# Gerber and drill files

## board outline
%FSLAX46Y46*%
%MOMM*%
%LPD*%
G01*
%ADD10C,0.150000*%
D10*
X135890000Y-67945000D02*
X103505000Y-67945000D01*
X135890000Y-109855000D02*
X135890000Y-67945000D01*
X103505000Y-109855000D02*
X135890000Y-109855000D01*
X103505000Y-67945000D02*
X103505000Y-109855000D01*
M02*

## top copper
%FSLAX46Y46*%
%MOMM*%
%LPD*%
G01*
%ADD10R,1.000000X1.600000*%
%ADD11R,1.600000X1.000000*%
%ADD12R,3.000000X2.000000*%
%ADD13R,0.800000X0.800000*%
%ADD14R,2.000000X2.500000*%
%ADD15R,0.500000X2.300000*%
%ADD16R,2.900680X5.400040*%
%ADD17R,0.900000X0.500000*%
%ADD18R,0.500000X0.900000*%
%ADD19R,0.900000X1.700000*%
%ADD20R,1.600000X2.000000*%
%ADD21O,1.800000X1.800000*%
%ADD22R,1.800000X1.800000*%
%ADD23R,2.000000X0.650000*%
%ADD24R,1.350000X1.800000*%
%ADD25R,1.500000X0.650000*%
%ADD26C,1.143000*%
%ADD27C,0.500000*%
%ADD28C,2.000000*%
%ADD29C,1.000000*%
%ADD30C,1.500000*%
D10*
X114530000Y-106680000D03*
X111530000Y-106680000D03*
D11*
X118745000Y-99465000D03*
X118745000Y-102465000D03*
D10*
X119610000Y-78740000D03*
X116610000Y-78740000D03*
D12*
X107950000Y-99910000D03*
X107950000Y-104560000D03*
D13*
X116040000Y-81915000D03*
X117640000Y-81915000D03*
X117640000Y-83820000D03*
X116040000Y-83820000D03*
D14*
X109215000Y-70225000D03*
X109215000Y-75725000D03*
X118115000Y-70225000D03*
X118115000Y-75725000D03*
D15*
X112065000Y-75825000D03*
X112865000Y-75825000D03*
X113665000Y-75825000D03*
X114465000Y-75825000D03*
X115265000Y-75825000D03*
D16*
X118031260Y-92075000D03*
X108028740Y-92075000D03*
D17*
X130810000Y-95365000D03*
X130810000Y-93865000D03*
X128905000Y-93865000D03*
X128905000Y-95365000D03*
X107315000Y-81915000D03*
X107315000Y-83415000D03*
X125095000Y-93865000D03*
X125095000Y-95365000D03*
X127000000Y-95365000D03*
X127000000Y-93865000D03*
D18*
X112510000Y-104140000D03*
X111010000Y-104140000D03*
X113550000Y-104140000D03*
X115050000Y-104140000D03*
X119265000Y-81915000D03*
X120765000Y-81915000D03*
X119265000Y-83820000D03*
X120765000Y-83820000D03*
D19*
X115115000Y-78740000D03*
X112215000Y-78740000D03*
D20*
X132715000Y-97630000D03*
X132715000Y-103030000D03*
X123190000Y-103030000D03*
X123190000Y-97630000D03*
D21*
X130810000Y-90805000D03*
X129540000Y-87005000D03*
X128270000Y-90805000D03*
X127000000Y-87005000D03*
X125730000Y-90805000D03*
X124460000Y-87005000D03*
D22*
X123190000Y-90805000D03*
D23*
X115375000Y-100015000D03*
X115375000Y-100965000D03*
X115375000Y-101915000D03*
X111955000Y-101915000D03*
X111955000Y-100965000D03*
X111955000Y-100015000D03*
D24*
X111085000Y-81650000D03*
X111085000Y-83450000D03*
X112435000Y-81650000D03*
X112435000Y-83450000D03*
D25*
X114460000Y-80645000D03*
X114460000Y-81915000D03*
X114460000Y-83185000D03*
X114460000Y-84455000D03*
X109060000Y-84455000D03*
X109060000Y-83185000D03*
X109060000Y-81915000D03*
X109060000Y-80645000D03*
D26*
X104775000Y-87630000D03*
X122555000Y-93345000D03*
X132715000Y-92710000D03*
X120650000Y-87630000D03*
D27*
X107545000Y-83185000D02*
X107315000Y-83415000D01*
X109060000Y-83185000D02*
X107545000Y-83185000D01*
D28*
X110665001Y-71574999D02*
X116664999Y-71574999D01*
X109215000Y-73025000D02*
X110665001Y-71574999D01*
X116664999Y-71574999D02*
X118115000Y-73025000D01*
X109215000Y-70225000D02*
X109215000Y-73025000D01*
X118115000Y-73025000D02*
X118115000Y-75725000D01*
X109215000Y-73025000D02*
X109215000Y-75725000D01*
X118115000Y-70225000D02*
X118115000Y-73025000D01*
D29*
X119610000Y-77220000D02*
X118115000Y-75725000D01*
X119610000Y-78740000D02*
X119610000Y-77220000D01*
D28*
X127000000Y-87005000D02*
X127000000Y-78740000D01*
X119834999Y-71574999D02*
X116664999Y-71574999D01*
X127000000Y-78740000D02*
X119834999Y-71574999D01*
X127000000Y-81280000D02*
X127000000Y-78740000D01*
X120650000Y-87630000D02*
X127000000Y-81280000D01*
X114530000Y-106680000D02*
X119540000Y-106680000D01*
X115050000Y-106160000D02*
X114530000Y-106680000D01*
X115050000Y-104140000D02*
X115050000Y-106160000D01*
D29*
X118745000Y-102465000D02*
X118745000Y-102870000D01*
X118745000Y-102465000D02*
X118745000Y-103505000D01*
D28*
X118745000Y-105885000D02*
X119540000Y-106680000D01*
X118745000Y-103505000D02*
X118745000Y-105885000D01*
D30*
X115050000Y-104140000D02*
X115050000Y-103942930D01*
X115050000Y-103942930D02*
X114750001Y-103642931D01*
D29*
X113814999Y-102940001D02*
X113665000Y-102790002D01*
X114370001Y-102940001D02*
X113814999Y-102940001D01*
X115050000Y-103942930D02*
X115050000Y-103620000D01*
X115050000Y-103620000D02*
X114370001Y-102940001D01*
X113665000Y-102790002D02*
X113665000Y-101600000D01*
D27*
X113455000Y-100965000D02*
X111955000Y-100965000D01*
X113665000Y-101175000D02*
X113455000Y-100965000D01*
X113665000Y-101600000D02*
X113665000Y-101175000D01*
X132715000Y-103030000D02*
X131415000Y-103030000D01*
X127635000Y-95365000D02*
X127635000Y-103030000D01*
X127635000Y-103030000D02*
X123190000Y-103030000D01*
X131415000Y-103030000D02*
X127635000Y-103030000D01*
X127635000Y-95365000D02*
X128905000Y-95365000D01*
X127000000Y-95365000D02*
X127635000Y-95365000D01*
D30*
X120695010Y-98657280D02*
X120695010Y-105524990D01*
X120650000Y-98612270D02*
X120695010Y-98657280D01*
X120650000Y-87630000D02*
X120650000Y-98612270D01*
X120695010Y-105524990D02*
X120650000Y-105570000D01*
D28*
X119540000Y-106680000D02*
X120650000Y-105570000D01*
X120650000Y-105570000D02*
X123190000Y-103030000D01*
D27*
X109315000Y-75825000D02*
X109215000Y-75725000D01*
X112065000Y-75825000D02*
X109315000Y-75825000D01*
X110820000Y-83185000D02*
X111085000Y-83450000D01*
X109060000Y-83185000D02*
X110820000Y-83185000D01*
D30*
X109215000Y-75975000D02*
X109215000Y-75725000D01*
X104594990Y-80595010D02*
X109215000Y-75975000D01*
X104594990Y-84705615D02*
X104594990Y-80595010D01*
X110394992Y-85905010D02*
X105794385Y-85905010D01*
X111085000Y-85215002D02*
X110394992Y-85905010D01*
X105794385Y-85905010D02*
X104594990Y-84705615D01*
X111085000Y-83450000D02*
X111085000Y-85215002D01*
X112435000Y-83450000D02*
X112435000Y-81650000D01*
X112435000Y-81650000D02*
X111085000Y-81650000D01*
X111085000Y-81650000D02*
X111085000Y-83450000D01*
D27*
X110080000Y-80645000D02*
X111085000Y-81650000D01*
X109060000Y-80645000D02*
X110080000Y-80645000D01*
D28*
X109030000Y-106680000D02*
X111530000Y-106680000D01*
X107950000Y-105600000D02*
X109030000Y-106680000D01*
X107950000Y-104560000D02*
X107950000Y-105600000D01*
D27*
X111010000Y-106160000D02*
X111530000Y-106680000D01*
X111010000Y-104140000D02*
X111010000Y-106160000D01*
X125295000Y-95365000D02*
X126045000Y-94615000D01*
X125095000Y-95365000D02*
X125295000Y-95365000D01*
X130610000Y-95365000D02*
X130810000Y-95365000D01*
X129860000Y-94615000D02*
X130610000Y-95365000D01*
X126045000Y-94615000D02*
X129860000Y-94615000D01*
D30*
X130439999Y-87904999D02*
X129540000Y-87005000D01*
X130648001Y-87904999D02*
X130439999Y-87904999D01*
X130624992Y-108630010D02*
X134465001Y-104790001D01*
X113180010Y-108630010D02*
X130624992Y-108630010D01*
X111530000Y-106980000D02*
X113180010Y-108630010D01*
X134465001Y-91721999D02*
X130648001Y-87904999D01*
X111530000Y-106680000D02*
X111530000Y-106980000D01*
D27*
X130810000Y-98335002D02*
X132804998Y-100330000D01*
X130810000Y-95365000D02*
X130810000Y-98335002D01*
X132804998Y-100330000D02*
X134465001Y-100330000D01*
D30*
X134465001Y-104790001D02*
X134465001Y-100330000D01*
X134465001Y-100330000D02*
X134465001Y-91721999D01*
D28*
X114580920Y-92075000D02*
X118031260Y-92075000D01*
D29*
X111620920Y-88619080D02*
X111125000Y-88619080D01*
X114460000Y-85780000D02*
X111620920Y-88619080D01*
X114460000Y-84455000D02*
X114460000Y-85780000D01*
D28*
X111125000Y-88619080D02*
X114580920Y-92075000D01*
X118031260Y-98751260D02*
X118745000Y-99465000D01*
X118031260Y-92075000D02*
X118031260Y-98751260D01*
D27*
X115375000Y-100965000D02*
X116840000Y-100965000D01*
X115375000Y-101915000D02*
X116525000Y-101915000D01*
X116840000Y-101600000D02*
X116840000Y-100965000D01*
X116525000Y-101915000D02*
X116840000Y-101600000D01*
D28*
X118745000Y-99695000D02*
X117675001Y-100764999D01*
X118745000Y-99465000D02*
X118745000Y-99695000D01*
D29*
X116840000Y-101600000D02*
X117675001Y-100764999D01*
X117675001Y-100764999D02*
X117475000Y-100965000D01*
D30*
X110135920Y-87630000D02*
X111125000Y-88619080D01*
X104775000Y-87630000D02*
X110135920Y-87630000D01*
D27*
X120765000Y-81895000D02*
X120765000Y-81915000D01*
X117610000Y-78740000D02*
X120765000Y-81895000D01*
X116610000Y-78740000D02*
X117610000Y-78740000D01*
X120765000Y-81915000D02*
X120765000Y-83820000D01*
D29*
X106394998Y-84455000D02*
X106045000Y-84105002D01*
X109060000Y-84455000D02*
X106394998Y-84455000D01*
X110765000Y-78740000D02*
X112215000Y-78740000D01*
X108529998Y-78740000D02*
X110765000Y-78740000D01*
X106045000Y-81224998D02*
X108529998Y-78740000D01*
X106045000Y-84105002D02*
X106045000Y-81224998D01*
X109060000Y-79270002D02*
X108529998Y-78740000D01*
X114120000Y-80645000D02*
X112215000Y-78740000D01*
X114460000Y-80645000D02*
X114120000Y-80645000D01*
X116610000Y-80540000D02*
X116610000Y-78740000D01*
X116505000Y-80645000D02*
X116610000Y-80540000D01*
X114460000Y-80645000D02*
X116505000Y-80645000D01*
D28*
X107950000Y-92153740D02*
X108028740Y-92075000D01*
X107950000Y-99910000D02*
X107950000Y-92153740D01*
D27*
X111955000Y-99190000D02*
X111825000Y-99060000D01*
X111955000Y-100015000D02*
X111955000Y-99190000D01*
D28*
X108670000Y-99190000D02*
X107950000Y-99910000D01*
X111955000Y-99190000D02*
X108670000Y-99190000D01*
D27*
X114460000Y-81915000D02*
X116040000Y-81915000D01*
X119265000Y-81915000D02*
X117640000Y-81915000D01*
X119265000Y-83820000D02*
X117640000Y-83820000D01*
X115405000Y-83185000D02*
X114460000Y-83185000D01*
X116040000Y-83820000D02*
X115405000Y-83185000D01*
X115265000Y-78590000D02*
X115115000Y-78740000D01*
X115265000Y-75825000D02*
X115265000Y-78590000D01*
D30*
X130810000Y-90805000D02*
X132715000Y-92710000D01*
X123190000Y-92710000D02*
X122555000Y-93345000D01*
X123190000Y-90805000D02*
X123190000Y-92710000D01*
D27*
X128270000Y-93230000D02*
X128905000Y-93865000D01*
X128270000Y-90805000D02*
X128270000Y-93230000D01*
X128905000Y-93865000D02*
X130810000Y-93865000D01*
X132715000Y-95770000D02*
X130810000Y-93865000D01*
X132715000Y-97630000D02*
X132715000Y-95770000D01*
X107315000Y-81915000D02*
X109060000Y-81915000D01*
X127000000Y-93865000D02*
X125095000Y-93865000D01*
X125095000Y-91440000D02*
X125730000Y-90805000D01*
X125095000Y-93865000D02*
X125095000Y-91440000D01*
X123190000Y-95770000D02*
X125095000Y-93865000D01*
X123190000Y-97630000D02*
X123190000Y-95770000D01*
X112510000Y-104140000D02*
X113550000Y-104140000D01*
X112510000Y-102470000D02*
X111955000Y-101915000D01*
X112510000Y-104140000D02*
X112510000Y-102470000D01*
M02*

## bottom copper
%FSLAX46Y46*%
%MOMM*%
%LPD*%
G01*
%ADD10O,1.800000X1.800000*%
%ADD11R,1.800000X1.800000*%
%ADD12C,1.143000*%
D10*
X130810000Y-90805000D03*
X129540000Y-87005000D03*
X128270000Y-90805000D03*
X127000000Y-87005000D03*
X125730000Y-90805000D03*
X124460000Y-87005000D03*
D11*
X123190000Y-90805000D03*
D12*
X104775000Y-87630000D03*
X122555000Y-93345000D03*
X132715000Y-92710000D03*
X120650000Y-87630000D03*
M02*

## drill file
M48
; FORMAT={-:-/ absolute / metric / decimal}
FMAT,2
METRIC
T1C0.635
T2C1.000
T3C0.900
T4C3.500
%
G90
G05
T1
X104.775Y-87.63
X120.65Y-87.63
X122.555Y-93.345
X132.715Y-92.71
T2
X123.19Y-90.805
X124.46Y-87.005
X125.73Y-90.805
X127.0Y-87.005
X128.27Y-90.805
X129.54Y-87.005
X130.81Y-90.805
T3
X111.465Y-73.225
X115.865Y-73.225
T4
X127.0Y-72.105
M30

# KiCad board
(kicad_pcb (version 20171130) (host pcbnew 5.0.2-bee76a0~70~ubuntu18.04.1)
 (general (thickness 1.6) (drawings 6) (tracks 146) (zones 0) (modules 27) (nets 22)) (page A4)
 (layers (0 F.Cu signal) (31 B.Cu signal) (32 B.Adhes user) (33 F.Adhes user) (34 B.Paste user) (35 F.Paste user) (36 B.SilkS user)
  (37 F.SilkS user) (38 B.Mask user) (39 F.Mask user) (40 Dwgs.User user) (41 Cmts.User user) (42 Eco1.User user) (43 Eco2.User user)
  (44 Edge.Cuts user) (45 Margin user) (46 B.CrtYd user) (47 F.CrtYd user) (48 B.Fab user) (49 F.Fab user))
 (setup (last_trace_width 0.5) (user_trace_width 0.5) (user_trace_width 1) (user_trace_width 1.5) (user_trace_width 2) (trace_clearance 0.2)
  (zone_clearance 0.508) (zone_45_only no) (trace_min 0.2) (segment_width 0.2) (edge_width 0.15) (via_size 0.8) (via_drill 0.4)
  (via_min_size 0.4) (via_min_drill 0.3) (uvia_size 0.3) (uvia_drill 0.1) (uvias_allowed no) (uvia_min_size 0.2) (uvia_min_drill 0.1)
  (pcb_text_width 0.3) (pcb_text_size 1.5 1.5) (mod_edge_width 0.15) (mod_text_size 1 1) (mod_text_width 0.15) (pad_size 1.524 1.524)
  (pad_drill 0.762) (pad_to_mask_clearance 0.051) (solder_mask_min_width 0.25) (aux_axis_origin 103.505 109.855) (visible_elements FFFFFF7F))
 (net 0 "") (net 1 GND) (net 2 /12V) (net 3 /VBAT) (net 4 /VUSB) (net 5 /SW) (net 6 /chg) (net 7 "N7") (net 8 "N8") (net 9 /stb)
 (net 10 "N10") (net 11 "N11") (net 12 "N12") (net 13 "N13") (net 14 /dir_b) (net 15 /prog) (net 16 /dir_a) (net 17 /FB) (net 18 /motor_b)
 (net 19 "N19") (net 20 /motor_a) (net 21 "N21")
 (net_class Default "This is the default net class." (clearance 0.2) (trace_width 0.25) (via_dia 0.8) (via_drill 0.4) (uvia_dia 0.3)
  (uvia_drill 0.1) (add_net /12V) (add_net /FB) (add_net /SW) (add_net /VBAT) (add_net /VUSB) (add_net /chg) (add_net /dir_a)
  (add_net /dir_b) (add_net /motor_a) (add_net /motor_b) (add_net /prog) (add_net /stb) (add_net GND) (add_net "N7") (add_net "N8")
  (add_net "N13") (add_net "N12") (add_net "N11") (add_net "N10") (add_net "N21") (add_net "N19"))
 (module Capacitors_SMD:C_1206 (layer F.Cu) (at 113.03 106.68)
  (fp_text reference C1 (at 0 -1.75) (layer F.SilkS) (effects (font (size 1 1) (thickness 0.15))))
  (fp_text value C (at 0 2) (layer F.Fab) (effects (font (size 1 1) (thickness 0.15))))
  (pad 2 smd rect (at 1.5 0) (size 1 1.6) (layers F.Cu F.Paste F.Mask) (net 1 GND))
  (pad 1 smd rect (at -1.5 0) (size 1 1.6) (layers F.Cu F.Paste F.Mask) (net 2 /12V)))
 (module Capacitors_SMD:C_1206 (layer F.Cu) (at 118.745 100.965 270)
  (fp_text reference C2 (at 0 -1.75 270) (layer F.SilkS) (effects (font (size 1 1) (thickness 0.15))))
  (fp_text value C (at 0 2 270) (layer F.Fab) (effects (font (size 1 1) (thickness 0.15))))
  (pad 1 smd rect (at -1.5 0 270) (size 1 1.6) (layers F.Cu F.Paste F.Mask) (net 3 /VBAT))
  (pad 2 smd rect (at 1.5 0 270) (size 1 1.6) (layers F.Cu F.Paste F.Mask) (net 1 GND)))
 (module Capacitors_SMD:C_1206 (layer F.Cu) (at 118.11 78.74)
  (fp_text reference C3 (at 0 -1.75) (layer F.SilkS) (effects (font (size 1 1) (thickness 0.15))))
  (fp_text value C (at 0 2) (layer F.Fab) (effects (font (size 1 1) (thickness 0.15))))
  (pad 2 smd rect (at 1.5 0) (size 1 1.6) (layers F.Cu F.Paste F.Mask) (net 1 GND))
  (pad 1 smd rect (at -1.5 0) (size 1 1.6) (layers F.Cu F.Paste F.Mask) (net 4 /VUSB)))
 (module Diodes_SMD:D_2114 (layer F.Cu) (at 107.95 102.235 90)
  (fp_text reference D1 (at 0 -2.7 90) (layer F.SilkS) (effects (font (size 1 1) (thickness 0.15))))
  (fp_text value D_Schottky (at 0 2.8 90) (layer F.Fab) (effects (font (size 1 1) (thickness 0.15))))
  (pad 2 smd rect (at 2.325 0 90) (size 2 3) (layers F.Cu F.Paste F.Mask) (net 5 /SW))
  (pad 1 smd rect (at -2.325 0 90) (size 2 3) (layers F.Cu F.Paste F.Mask) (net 2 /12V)))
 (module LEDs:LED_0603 (layer F.Cu) (at 116.84 81.915)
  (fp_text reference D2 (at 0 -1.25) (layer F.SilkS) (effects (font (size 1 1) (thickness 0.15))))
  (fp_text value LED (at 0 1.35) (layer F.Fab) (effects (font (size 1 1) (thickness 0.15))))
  (pad 1 smd rect (at -0.8 0 180) (size 0.8 0.8) (layers F.Cu F.Paste F.Mask) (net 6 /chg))
  (pad 2 smd rect (at 0.8 0 180) (size 0.8 0.8) (layers F.Cu F.Paste F.Mask) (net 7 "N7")))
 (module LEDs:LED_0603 (layer F.Cu) (at 116.84 83.82)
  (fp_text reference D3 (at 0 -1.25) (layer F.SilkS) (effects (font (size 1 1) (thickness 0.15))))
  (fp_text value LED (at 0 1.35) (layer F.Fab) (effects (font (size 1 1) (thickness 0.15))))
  (pad 2 smd rect (at 0.8 0 180) (size 0.8 0.8) (layers F.Cu F.Paste F.Mask) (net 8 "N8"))
  (pad 1 smd rect (at -0.8 0 180) (size 0.8 0.8) (layers F.Cu F.Paste F.Mask) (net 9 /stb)))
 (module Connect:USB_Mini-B (layer F.Cu) (at 113.665 73.025 270)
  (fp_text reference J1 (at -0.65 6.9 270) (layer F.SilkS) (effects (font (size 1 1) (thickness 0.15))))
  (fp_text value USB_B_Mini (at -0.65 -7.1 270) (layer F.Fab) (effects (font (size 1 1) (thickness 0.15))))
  (pad "" np_thru_hole circle (at 0.2 2.2 270) (size 0.9 0.9) (drill 0.9) (layers *.Cu *.Mask))
  (pad "" np_thru_hole circle (at 0.2 -2.2 270) (size 0.9 0.9) (drill 0.9) (layers *.Cu *.Mask))
  (pad 6 smd rect (at -2.8 4.45 270) (size 2.5 2) (layers F.Cu F.Paste F.Mask) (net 1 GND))
  (pad 6 smd rect (at 2.7 4.45 270) (size 2.5 2) (layers F.Cu F.Paste F.Mask) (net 1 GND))
  (pad 6 smd rect (at -2.8 -4.45 270) (size 2.5 2) (layers F.Cu F.Paste F.Mask) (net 1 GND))
  (pad 6 smd rect (at 2.7 -4.45 270) (size 2.5 2) (layers F.Cu F.Paste F.Mask) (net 1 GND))
  (pad 5 smd rect (at 2.8 1.6 270) (size 2.3 0.5) (layers F.Cu F.Paste F.Mask) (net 1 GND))
  (pad 4 smd rect (at 2.8 0.8 270) (size 2.3 0.5) (layers F.Cu F.Paste F.Mask) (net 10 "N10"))
  (pad 3 smd rect (at 2.8 0 270) (size 2.3 0.5) (layers F.Cu F.Paste F.Mask) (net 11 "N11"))
  (pad 2 smd rect (at 2.8 -0.8 270) (size 2.3 0.5) (layers F.Cu F.Paste F.Mask) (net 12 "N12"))
  (pad 1 smd rect (at 2.8 -1.6 270) (size 2.3 0.5) (layers F.Cu F.Paste F.Mask) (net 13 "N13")))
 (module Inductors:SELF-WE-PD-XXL (layer F.Cu) (at 113.03 92.075)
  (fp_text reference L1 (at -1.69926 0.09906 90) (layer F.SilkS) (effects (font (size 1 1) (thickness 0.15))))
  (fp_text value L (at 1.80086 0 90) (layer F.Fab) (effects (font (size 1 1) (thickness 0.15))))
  (pad 2 smd rect (at 5.00126 0) (size 2.90068 5.40004) (layers F.Cu F.Paste F.Mask) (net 3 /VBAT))
  (pad 1 smd rect (at -5.00126 0) (size 2.90068 5.40004) (layers F.Cu F.Paste F.Mask) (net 5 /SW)))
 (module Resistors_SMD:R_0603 (layer F.Cu) (at 130.81 94.615 90)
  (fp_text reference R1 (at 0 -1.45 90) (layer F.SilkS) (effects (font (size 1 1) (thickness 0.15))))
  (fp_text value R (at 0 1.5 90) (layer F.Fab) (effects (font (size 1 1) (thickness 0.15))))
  (pad 1 smd rect (at -0.75 0 90) (size 0.5 0.9) (layers F.Cu F.Paste F.Mask) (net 2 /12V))
  (pad 2 smd rect (at 0.75 0 90) (size 0.5 0.9) (layers F.Cu F.Paste F.Mask) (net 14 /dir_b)))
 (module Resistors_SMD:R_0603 (layer F.Cu) (at 128.905 94.615 270)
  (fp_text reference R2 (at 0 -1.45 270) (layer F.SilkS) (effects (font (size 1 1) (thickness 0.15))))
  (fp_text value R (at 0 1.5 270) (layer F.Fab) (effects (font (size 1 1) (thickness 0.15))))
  (pad 1 smd rect (at -0.75 0 270) (size 0.5 0.9) (layers F.Cu F.Paste F.Mask) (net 14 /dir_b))
  (pad 2 smd rect (at 0.75 0 270) (size 0.5 0.9) (layers F.Cu F.Paste F.Mask) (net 1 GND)))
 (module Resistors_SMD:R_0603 (layer F.Cu) (at 107.315 82.665 270)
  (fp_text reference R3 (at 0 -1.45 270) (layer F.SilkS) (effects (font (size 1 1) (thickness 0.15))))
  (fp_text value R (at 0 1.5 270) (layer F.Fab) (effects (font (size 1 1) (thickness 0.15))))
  (pad 1 smd rect (at -0.75 0 270) (size 0.5 0.9) (layers F.Cu F.Paste F.Mask) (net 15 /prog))
  (pad 2 smd rect (at 0.75 0 270) (size 0.5 0.9) (layers F.Cu F.Paste F.Mask) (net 1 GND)))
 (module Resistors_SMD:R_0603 (layer F.Cu) (at 125.095 94.615 90)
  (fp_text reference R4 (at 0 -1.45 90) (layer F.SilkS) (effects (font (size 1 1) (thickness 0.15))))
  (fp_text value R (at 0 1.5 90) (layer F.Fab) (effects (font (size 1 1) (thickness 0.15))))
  (pad 2 smd rect (at 0.75 0 90) (size 0.5 0.9) (layers F.Cu F.Paste F.Mask) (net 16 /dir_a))
  (pad 1 smd rect (at -0.75 0 90) (size 0.5 0.9) (layers F.Cu F.Paste F.Mask) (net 2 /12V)))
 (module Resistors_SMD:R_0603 (layer F.Cu) (at 127 94.615 270)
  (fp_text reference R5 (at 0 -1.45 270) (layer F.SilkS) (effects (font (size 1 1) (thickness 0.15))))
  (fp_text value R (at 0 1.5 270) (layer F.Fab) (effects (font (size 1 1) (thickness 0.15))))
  (pad 2 smd rect (at 0.75 0 270) (size 0.5 0.9) (layers F.Cu F.Paste F.Mask) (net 1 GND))
  (pad 1 smd rect (at -0.75 0 270) (size 0.5 0.9) (layers F.Cu F.Paste F.Mask) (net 16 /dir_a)))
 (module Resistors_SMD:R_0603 (layer F.Cu) (at 111.76 104.14)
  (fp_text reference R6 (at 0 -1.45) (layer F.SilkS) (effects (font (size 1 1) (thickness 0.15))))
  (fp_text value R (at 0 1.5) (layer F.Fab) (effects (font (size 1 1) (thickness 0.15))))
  (pad 2 smd rect (at 0.75 0) (size 0.5 0.9) (layers F.Cu F.Paste F.Mask) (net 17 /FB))
  (pad 1 smd rect (at -0.75 0) (size 0.5 0.9) (layers F.Cu F.Paste F.Mask) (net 2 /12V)))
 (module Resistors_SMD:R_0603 (layer F.Cu) (at 114.3 104.14)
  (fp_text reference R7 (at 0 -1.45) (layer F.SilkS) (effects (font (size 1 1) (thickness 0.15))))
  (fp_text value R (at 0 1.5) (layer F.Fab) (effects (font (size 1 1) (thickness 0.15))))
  (pad 1 smd rect (at -0.75 0) (size 0.5 0.9) (layers F.Cu F.Paste F.Mask) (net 17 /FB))
  (pad 2 smd rect (at 0.75 0) (size 0.5 0.9) (layers F.Cu F.Paste F.Mask) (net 1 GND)))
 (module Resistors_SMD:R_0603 (layer F.Cu) (at 120.015 81.915 180)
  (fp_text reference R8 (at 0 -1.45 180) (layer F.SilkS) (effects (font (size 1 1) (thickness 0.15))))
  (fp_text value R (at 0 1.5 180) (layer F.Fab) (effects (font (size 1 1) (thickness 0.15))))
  (pad 2 smd rect (at 0.75 0 180) (size 0.5 0.9) (layers F.Cu F.Paste F.Mask) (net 7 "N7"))
  (pad 1 smd rect (at -0.75 0 180) (size 0.5 0.9) (layers F.Cu F.Paste F.Mask) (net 4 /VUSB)))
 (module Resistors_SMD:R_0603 (layer F.Cu) (at 120.015 83.82 180)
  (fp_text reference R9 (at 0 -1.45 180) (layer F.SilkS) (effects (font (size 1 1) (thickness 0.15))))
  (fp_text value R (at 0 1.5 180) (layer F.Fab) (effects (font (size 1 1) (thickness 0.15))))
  (pad 2 smd rect (at 0.75 0 180) (size 0.5 0.9) (layers F.Cu F.Paste F.Mask) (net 8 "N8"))
  (pad 1 smd rect (at -0.75 0 180) (size 0.5 0.9) (layers F.Cu F.Paste F.Mask) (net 4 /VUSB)))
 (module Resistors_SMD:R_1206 (layer F.Cu) (at 113.665 78.74)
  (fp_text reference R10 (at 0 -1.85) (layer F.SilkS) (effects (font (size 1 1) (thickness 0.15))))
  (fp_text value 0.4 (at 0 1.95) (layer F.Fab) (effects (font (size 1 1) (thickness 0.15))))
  (pad 2 smd rect (at 1.45 0) (size 0.9 1.7) (layers F.Cu F.Paste F.Mask) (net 13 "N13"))
  (pad 1 smd rect (at -1.45 0) (size 0.9 1.7) (layers F.Cu F.Paste F.Mask) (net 4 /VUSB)))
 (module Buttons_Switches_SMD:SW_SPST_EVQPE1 (layer F.Cu) (at 132.715 100.33 270)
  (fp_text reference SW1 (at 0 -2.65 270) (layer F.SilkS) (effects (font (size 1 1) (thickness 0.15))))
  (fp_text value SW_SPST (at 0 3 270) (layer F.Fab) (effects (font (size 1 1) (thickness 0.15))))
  (pad 1 smd rect (at -2.7 0 270) (size 2 1.6) (layers F.Cu F.Paste F.Mask) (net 14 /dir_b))
  (pad 2 smd rect (at 2.7 0 270) (size 2 1.6) (layers F.Cu F.Paste F.Mask) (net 1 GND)))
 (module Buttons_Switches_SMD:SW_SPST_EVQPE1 (layer F.Cu) (at 123.19 100.33 270)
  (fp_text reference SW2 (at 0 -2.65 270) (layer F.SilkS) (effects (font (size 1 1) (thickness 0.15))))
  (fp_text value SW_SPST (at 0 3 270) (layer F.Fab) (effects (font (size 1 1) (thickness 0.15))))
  (pad 2 smd rect (at 2.7 0 270) (size 2 1.6) (layers F.Cu F.Paste F.Mask) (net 1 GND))
  (pad 1 smd rect (at -2.7 0 270) (size 2 1.6) (layers F.Cu F.Paste F.Mask) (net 16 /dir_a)))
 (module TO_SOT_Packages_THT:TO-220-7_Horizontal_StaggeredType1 (layer F.Cu) (at 123.19 90.805)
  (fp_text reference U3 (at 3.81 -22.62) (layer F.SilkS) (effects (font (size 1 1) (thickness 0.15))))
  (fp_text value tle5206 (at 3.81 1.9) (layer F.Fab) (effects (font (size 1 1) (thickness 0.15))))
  (pad 7 thru_hole oval (at 7.62 0) (size 1.8 1.8) (drill 1) (layers *.Cu *.Mask) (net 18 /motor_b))
  (pad 6 thru_hole oval (at 6.35 -3.8) (size 1.8 1.8) (drill 1) (layers *.Cu *.Mask) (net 2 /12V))
  (pad 5 thru_hole oval (at 5.08 0) (size 1.8 1.8) (drill 1) (layers *.Cu *.Mask) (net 14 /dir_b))
  (pad 4 thru_hole oval (at 3.81 -3.8) (size 1.8 1.8) (drill 1) (layers *.Cu *.Mask) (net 1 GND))
  (pad 3 thru_hole oval (at 2.54 0) (size 1.8 1.8) (drill 1) (layers *.Cu *.Mask) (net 16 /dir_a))
  (pad 2 thru_hole oval (at 1.27 -3.8) (size 1.8 1.8) (drill 1) (layers *.Cu *.Mask) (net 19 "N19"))
  (pad 1 thru_hole rect (at 0 0) (size 1.8 1.8) (drill 1) (layers *.Cu *.Mask) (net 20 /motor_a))
  (pad 0 np_thru_hole oval (at 3.81 -18.7) (size 3.5 3.5) (drill 3.5) (layers *.Cu *.Mask)))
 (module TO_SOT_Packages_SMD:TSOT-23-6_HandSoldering (layer F.Cu) (at 113.665 100.965)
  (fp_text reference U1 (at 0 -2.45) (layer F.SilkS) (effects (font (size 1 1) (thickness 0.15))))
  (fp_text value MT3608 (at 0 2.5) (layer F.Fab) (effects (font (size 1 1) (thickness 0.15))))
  (pad 6 smd rect (at 1.71 -0.95) (size 2 0.65) (layers F.Cu F.Paste F.Mask) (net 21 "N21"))
  (pad 5 smd rect (at 1.71 0) (size 2 0.65) (layers F.Cu F.Paste F.Mask) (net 3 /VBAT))
  (pad 4 smd rect (at 1.71 0.95) (size 2 0.65) (layers F.Cu F.Paste F.Mask) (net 3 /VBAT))
  (pad 3 smd rect (at -1.71 0.95) (size 2 0.65) (layers F.Cu F.Paste F.Mask) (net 17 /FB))
  (pad 2 smd rect (at -1.71 0) (size 2 0.65) (layers F.Cu F.Paste F.Mask) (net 1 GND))
  (pad 1 smd rect (at -1.71 -0.95) (size 2 0.65) (layers F.Cu F.Paste F.Mask) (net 5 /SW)))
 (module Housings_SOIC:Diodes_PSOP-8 (layer F.Cu) (at 111.76 82.55)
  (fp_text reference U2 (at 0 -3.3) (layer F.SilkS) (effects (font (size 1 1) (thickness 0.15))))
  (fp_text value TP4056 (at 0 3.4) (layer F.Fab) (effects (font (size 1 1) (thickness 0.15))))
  (pad 9 smd rect (at -0.675 -0.9) (size 1.35 1.8) (layers F.Cu F.Paste F.Mask) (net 1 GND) (solder_paste_margin_ratio -0.2))
  (pad 9 smd rect (at -0.675 0.9) (size 1.35 1.8) (layers F.Cu F.Paste F.Mask) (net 1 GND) (solder_paste_margin_ratio -0.2))
  (pad 9 smd rect (at 0.675 -0.9) (size 1.35 1.8) (layers F.Cu F.Paste F.Mask) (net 1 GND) (solder_paste_margin_ratio -0.2))
  (pad 9 smd rect (at 0.675 0.9) (size 1.35 1.8) (layers F.Cu F.Paste F.Mask) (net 1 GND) (solder_paste_margin_ratio -0.2))
  (pad 8 smd rect (at 2.7 -1.905) (size 1.5 0.65) (layers F.Cu F.Paste F.Mask) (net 4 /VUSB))
  (pad 7 smd rect (at 2.7 -0.635) (size 1.5 0.65) (layers F.Cu F.Paste F.Mask) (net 6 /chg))
  (pad 6 smd rect (at 2.7 0.635) (size 1.5 0.65) (layers F.Cu F.Paste F.Mask) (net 9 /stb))
  (pad 5 smd rect (at 2.7 1.905) (size 1.5 0.65) (layers F.Cu F.Paste F.Mask) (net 3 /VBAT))
  (pad 4 smd rect (at -2.7 1.905) (size 1.5 0.65) (layers F.Cu F.Paste F.Mask) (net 4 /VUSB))
  (pad 3 smd rect (at -2.7 0.635) (size 1.5 0.65) (layers F.Cu F.Paste F.Mask) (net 1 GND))
  (pad 2 smd rect (at -2.7 -0.635) (size 1.5 0.65) (layers F.Cu F.Paste F.Mask) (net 15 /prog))
  (pad 1 smd rect (at -2.7 -1.905) (size 1.5 0.65) (layers F.Cu F.Paste F.Mask) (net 1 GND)))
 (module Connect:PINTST (layer F.Cu) (at 104.775 87.63)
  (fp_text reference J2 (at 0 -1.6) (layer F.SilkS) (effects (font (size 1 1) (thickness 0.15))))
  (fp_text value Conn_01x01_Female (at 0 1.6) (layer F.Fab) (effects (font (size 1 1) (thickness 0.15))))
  (pad 1 thru_hole circle (at 0 0) (size 1.143 1.143) (drill 0.635) (layers *.Cu *.Mask) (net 3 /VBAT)))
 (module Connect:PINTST (layer F.Cu) (at 122.555 93.345)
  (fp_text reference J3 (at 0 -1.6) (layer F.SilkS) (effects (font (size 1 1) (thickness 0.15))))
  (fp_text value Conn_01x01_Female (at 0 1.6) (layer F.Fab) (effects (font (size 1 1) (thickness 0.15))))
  (pad 1 thru_hole circle (at 0 0) (size 1.143 1.143) (drill 0.635) (layers *.Cu *.Mask) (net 20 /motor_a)))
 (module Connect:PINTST (layer F.Cu) (at 132.715 92.71)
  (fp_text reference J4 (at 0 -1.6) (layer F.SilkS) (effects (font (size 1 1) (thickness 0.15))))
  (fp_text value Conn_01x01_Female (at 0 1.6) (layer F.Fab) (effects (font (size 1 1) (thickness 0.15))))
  (pad 1 thru_hole circle (at 0 0) (size 1.143 1.143) (drill 0.635) (layers *.Cu *.Mask) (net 18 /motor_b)))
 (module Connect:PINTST (layer F.Cu) (at 120.65 87.63)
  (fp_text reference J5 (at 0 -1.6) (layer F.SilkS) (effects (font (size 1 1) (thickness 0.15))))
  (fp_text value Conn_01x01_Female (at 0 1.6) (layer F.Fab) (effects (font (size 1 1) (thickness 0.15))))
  (pad 1 thru_hole circle (at 0 0) (size 1.143 1.143) (drill 0.635) (layers *.Cu *.Mask) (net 1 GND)))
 (gr_line (start 135.89 67.945) (end 103.505 67.945) (layer Edge.Cuts) (width 0.15))
 (gr_line (start 135.89 109.855) (end 135.89 67.945) (layer Edge.Cuts) (width 0.15))
 (gr_line (start 103.505 109.855) (end 135.89 109.855) (layer Edge.Cuts) (width 0.15))
 (gr_line (start 103.505 67.945) (end 103.505 109.855) (layer Edge.Cuts) (width 0.15))
 (segment (start 107.545 83.185) (end 107.315 83.415) (width 0.5) (layer F.Cu) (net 1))
 (segment (start 109.06 83.185) (end 107.545 83.185) (width 0.5) (layer F.Cu) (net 1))
 (segment (start 110.665001 71.574999) (end 116.664999 71.574999) (width 2) (layer F.Cu) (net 1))
 (segment (start 109.215 73.025) (end 110.665001 71.574999) (width 2) (layer F.Cu) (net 1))
 (segment (start 116.664999 71.574999) (end 118.115 73.025) (width 2) (layer F.Cu) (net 1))
 (segment (start 109.215 70.225) (end 109.215 73.025) (width 2) (layer F.Cu) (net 1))
 (segment (start 118.115 73.025) (end 118.115 75.725) (width 2) (layer F.Cu) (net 1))
 (segment (start 109.215 73.025) (end 109.215 75.725) (width 2) (layer F.Cu) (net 1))
 (segment (start 118.115 70.225) (end 118.115 73.025) (width 2) (layer F.Cu) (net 1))
 (segment (start 119.61 77.22) (end 118.115 75.725) (width 1) (layer F.Cu) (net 1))
 (segment (start 119.61 78.74) (end 119.61 77.22) (width 1) (layer F.Cu) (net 1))
 (segment (start 127 87.005) (end 127 78.74) (width 2) (layer F.Cu) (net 1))
 (segment (start 119.834999 71.574999) (end 116.664999 71.574999) (width 2) (layer F.Cu) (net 1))
 (segment (start 127 78.74) (end 119.834999 71.574999) (width 2) (layer F.Cu) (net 1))
 (segment (start 127 81.28) (end 127 78.74) (width 2) (layer F.Cu) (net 1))
 (segment (start 120.65 87.63) (end 127 81.28) (width 2) (layer F.Cu) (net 1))
 (segment (start 114.53 106.68) (end 119.54 106.68) (width 2) (layer F.Cu) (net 1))
 (segment (start 115.05 106.16) (end 114.53 106.68) (width 2) (layer F.Cu) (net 1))
 (segment (start 115.05 104.14) (end 115.05 106.16) (width 2) (layer F.Cu) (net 1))
 (segment (start 118.745 102.465) (end 118.745 102.87) (width 1) (layer F.Cu) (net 1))
 (segment (start 118.745 102.465) (end 118.745 103.505) (width 1) (layer F.Cu) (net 1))
 (segment (start 118.745 105.885) (end 119.54 106.68) (width 2) (layer F.Cu) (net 1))
 (segment (start 118.745 103.505) (end 118.745 105.885) (width 2) (layer F.Cu) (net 1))
 (segment (start 115.05 104.14) (end 115.05 103.94293) (width 1.5) (layer F.Cu) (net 1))
 (segment (start 115.05 103.94293) (end 114.750001 103.642931) (width 1.5) (layer F.Cu) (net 1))
 (segment (start 113.814999 102.940001) (end 113.665 102.790002) (width 1) (layer F.Cu) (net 1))
 (segment (start 114.370001 102.940001) (end 113.814999 102.940001) (width 1) (layer F.Cu) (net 1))
 (segment (start 115.05 103.94293) (end 115.05 103.62) (width 1) (layer F.Cu) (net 1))
 (segment (start 115.05 103.62) (end 114.370001 102.940001) (width 1) (layer F.Cu) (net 1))
 (segment (start 113.665 102.790002) (end 113.665 101.6) (width 1) (layer F.Cu) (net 1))
 (segment (start 113.455 100.965) (end 111.955 100.965) (width 0.5) (layer F.Cu) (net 1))
 (segment (start 113.665 101.175) (end 113.455 100.965) (width 0.5) (layer F.Cu) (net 1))
 (segment (start 113.665 101.6) (end 113.665 101.175) (width 0.5) (layer F.Cu) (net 1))
 (segment (start 132.715 103.03) (end 131.415 103.03) (width 0.5) (layer F.Cu) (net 1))
 (segment (start 127.635 95.365) (end 127.635 103.03) (width 0.5) (layer F.Cu) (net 1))
 (segment (start 127.635 103.03) (end 123.19 103.03) (width 0.5) (layer F.Cu) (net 1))
 (segment (start 131.415 103.03) (end 127.635 103.03) (width 0.5) (layer F.Cu) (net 1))
 (segment (start 127.635 95.365) (end 128.905 95.365) (width 0.5) (layer F.Cu) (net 1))
 (segment (start 127 95.365) (end 127.635 95.365) (width 0.5) (layer F.Cu) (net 1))
 (segment (start 120.69501 98.65728) (end 120.69501 105.52499) (width 1.5) (layer F.Cu) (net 1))
 (segment (start 120.65 98.61227) (end 120.69501 98.65728) (width 1.5) (layer F.Cu) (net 1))
 (segment (start 120.65 87.63) (end 120.65 98.61227) (width 1.5) (layer F.Cu) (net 1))
 (segment (start 120.69501 105.52499) (end 120.65 105.57) (width 1.5) (layer F.Cu) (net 1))
 (segment (start 119.54 106.68) (end 120.65 105.57) (width 2) (layer F.Cu) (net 1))
 (segment (start 120.65 105.57) (end 123.19 103.03) (width 2) (layer F.Cu) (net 1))
 (segment (start 109.315 75.825) (end 109.215 75.725) (width 0.5) (layer F.Cu) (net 1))
 (segment (start 112.065 75.825) (end 109.315 75.825) (width 0.5) (layer F.Cu) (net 1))
 (segment (start 110.82 83.185) (end 111.085 83.45) (width 0.5) (layer F.Cu) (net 1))
 (segment (start 109.06 83.185) (end 110.82 83.185) (width 0.5) (layer F.Cu) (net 1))
 (segment (start 109.215 75.975) (end 109.215 75.725) (width 1.5) (layer F.Cu) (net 1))
 (segment (start 104.59499 80.59501) (end 109.215 75.975) (width 1.5) (layer F.Cu) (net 1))
 (segment (start 104.59499 84.705615) (end 104.59499 80.59501) (width 1.5) (layer F.Cu) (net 1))
 (segment (start 110.394992 85.90501) (end 105.794385 85.90501) (width 1.5) (layer F.Cu) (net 1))
 (segment (start 111.085 85.215002) (end 110.394992 85.90501) (width 1.5) (layer F.Cu) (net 1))
 (segment (start 105.794385 85.90501) (end 104.59499 84.705615) (width 1.5) (layer F.Cu) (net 1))
 (segment (start 111.085 83.45) (end 111.085 85.215002) (width 1.5) (layer F.Cu) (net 1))
 (segment (start 112.435 83.45) (end 112.435 81.65) (width 1.5) (layer F.Cu) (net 1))
 (segment (start 112.435 81.65) (end 111.085 81.65) (width 1.5) (layer F.Cu) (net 1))
 (segment (start 111.085 81.65) (end 111.085 83.45) (width 1.5) (layer F.Cu) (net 1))
 (segment (start 110.08 80.645) (end 111.085 81.65) (width 0.5) (layer F.Cu) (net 1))
 (segment (start 109.06 80.645) (end 110.08 80.645) (width 0.5) (layer F.Cu) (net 1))
 (segment (start 109.03 106.68) (end 111.53 106.68) (width 2) (layer F.Cu) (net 2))
 (segment (start 107.95 105.6) (end 109.03 106.68) (width 2) (layer F.Cu) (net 2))
 (segment (start 107.95 104.56) (end 107.95 105.6) (width 2) (layer F.Cu) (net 2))
 (segment (start 111.01 106.16) (end 111.53 106.68) (width 0.5) (layer F.Cu) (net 2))
 (segment (start 111.01 104.14) (end 111.01 106.16) (width 0.5) (layer F.Cu) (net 2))
 (segment (start 125.295 95.365) (end 126.045 94.615) (width 0.5) (layer F.Cu) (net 2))
 (segment (start 125.095 95.365) (end 125.295 95.365) (width 0.5) (layer F.Cu) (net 2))
 (segment (start 130.61 95.365) (end 130.81 95.365) (width 0.5) (layer F.Cu) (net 2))
 (segment (start 129.86 94.615) (end 130.61 95.365) (width 0.5) (layer F.Cu) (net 2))
 (segment (start 126.045 94.615) (end 129.86 94.615) (width 0.5) (layer F.Cu) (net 2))
 (segment (start 130.439999 87.904999) (end 129.54 87.005) (width 1.5) (layer F.Cu) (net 2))
 (segment (start 130.648001 87.904999) (end 130.439999 87.904999) (width 1.5) (layer F.Cu) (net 2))
 (segment (start 130.624992 108.63001) (end 134.465001 104.790001) (width 1.5) (layer F.Cu) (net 2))
 (segment (start 113.18001 108.63001) (end 130.624992 108.63001) (width 1.5) (layer F.Cu) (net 2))
 (segment (start 111.53 106.98) (end 113.18001 108.63001) (width 1.5) (layer F.Cu) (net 2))
 (segment (start 134.465001 91.721999) (end 130.648001 87.904999) (width 1.5) (layer F.Cu) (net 2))
 (segment (start 111.53 106.68) (end 111.53 106.98) (width 1.5) (layer F.Cu) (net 2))
 (segment (start 130.81 98.335002) (end 132.804998 100.33) (width 0.5) (layer F.Cu) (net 2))
 (segment (start 130.81 95.365) (end 130.81 98.335002) (width 0.5) (layer F.Cu) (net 2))
 (segment (start 132.804998 100.33) (end 134.465001 100.33) (width 0.5) (layer F.Cu) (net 2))
 (segment (start 134.465001 104.790001) (end 134.465001 100.33) (width 1.5) (layer F.Cu) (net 2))
 (segment (start 134.465001 100.33) (end 134.465001 91.721999) (width 1.5) (layer F.Cu) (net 2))
 (segment (start 114.58092 92.075) (end 118.03126 92.075) (width 2) (layer F.Cu) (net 3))
 (segment (start 111.62092 88.61908) (end 111.125 88.61908) (width 1) (layer F.Cu) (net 3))
 (segment (start 114.46 85.78) (end 111.62092 88.61908) (width 1) (layer F.Cu) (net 3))
 (segment (start 114.46 84.455) (end 114.46 85.78) (width 1) (layer F.Cu) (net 3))
 (segment (start 111.125 88.61908) (end 114.58092 92.075) (width 2) (layer F.Cu) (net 3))
 (segment (start 118.03126 98.75126) (end 118.745 99.465) (width 2) (layer F.Cu) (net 3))
 (segment (start 118.03126 92.075) (end 118.03126 98.75126) (width 2) (layer F.Cu) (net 3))
 (segment (start 115.375 100.965) (end 116.84 100.965) (width 0.5) (layer F.Cu) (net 3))
 (segment (start 115.375 101.915) (end 116.525 101.915) (width 0.5) (layer F.Cu) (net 3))
 (segment (start 116.84 101.6) (end 116.84 100.965) (width 0.5) (layer F.Cu) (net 3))
 (segment (start 116.525 101.915) (end 116.84 101.6) (width 0.5) (layer F.Cu) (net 3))
 (segment (start 118.745 99.695) (end 117.675001 100.764999) (width 2) (layer F.Cu) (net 3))
 (segment (start 118.745 99.465) (end 118.745 99.695) (width 2) (layer F.Cu) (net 3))
 (segment (start 116.84 101.6) (end 117.675001 100.764999) (width 1) (layer F.Cu) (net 3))
 (segment (start 117.675001 100.764999) (end 117.475 100.965) (width 1) (layer F.Cu) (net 3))
 (segment (start 110.13592 87.63) (end 111.125 88.61908) (width 1.5) (layer F.Cu) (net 3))
 (segment (start 104.775 87.63) (end 110.13592 87.63) (width 1.5) (layer F.Cu) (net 3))
 (segment (start 120.765 81.895) (end 120.765 81.915) (width 0.5) (layer F.Cu) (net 4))
 (segment (start 117.61 78.74) (end 120.765 81.895) (width 0.5) (layer F.Cu) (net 4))
 (segment (start 116.61 78.74) (end 117.61 78.74) (width 0.5) (layer F.Cu) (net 4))
 (segment (start 120.765 81.915) (end 120.765 83.82) (width 0.5) (layer F.Cu) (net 4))
 (segment (start 106.394998 84.455) (end 106.045 84.105002) (width 1) (layer F.Cu) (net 4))
 (segment (start 109.06 84.455) (end 106.394998 84.455) (width 1) (layer F.Cu) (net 4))
 (segment (start 110.765 78.74) (end 112.215 78.74) (width 1) (layer F.Cu) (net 4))
 (segment (start 108.529998 78.74) (end 110.765 78.74) (width 1) (layer F.Cu) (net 4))
 (segment (start 106.045 81.224998) (end 108.529998 78.74) (width 1) (layer F.Cu) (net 4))
 (segment (start 106.045 84.105002) (end 106.045 81.224998) (width 1) (layer F.Cu) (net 4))
 (segment (start 109.06 79.270002) (end 108.529998 78.74) (width 1) (layer F.Cu) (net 4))
 (segment (start 114.12 80.645) (end 112.215 78.74) (width 1) (layer F.Cu) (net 4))
 (segment (start 114.46 80.645) (end 114.12 80.645) (width 1) (layer F.Cu) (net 4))
 (segment (start 116.61 80.54) (end 116.61 78.74) (width 1) (layer F.Cu) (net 4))
 (segment (start 116.505 80.645) (end 116.61 80.54) (width 1) (layer F.Cu) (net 4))
 (segment (start 114.46 80.645) (end 116.505 80.645) (width 1) (layer F.Cu) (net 4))
 (segment (start 107.95 92.15374) (end 108.02874 92.075) (width 2) (layer F.Cu) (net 5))
 (segment (start 107.95 99.91) (end 107.95 92.15374) (width 2) (layer F.Cu) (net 5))
 (segment (start 111.955 99.19) (end 111.825 99.06) (width 0.5) (layer F.Cu) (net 5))
 (segment (start 111.955 100.015) (end 111.955 99.19) (width 0.5) (layer F.Cu) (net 5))
 (segment (start 108.67 99.19) (end 107.95 99.91) (width 2) (layer F.Cu) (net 5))
 (segment (start 111.955 99.19) (end 108.67 99.19) (width 2) (layer F.Cu) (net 5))
 (segment (start 114.46 81.915) (end 116.04 81.915) (width 0.5) (layer F.Cu) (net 6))
 (segment (start 119.265 81.915) (end 117.64 81.915) (width 0.5) (layer F.Cu) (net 7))
 (segment (start 119.265 83.82) (end 117.64 83.82) (width 0.5) (layer F.Cu) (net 8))
 (segment (start 115.405 83.185) (end 114.46 83.185) (width 0.5) (layer F.Cu) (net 9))
 (segment (start 116.04 83.82) (end 115.405 83.185) (width 0.5) (layer F.Cu) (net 9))
 (segment (start 115.265 78.59) (end 115.115 78.74) (width 0.5) (layer F.Cu) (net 13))
 (segment (start 115.265 75.825) (end 115.265 78.59) (width 0.5) (layer F.Cu) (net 13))
 (segment (start 130.81 90.805) (end 132.715 92.71) (width 1.5) (layer F.Cu) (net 18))
 (segment (start 123.19 92.71) (end 122.555 93.345) (width 1.5) (layer F.Cu) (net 20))
 (segment (start 123.19 90.805) (end 123.19 92.71) (width 1.5) (layer F.Cu) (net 20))
 (segment (start 128.27 93.23) (end 128.905 93.865) (width 0.5) (layer F.Cu) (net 14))
 (segment (start 128.27 90.805) (end 128.27 93.23) (width 0.5) (layer F.Cu) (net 14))
 (segment (start 128.905 93.865) (end 130.81 93.865) (width 0.5) (layer F.Cu) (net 14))
 (segment (start 132.715 95.77) (end 130.81 93.865) (width 0.5) (layer F.Cu) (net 14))
 (segment (start 132.715 97.63) (end 132.715 95.77) (width 0.5) (layer F.Cu) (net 14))
 (segment (start 107.315 81.915) (end 109.06 81.915) (width 0.5) (layer F.Cu) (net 15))
 (segment (start 127 93.865) (end 125.095 93.865) (width 0.5) (layer F.Cu) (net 16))
 (segment (start 125.095 91.44) (end 125.73 90.805) (width 0.5) (layer F.Cu) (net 16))
 (segment (start 125.095 93.865) (end 125.095 91.44) (width 0.5) (layer F.Cu) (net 16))
 (segment (start 123.19 95.77) (end 125.095 93.865) (width 0.5) (layer F.Cu) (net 16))
 (segment (start 123.19 97.63) (end 123.19 95.77) (width 0.5) (layer F.Cu) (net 16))
 (segment (start 112.51 104.14) (end 113.55 104.14) (width 0.5) (layer F.Cu) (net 17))
 (segment (start 112.51 102.47) (end 111.955 101.915) (width 0.5) (layer F.Cu) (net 17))
 (segment (start 112.51 104.14) (end 112.51 102.47) (width 0.5) (layer F.Cu) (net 17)))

